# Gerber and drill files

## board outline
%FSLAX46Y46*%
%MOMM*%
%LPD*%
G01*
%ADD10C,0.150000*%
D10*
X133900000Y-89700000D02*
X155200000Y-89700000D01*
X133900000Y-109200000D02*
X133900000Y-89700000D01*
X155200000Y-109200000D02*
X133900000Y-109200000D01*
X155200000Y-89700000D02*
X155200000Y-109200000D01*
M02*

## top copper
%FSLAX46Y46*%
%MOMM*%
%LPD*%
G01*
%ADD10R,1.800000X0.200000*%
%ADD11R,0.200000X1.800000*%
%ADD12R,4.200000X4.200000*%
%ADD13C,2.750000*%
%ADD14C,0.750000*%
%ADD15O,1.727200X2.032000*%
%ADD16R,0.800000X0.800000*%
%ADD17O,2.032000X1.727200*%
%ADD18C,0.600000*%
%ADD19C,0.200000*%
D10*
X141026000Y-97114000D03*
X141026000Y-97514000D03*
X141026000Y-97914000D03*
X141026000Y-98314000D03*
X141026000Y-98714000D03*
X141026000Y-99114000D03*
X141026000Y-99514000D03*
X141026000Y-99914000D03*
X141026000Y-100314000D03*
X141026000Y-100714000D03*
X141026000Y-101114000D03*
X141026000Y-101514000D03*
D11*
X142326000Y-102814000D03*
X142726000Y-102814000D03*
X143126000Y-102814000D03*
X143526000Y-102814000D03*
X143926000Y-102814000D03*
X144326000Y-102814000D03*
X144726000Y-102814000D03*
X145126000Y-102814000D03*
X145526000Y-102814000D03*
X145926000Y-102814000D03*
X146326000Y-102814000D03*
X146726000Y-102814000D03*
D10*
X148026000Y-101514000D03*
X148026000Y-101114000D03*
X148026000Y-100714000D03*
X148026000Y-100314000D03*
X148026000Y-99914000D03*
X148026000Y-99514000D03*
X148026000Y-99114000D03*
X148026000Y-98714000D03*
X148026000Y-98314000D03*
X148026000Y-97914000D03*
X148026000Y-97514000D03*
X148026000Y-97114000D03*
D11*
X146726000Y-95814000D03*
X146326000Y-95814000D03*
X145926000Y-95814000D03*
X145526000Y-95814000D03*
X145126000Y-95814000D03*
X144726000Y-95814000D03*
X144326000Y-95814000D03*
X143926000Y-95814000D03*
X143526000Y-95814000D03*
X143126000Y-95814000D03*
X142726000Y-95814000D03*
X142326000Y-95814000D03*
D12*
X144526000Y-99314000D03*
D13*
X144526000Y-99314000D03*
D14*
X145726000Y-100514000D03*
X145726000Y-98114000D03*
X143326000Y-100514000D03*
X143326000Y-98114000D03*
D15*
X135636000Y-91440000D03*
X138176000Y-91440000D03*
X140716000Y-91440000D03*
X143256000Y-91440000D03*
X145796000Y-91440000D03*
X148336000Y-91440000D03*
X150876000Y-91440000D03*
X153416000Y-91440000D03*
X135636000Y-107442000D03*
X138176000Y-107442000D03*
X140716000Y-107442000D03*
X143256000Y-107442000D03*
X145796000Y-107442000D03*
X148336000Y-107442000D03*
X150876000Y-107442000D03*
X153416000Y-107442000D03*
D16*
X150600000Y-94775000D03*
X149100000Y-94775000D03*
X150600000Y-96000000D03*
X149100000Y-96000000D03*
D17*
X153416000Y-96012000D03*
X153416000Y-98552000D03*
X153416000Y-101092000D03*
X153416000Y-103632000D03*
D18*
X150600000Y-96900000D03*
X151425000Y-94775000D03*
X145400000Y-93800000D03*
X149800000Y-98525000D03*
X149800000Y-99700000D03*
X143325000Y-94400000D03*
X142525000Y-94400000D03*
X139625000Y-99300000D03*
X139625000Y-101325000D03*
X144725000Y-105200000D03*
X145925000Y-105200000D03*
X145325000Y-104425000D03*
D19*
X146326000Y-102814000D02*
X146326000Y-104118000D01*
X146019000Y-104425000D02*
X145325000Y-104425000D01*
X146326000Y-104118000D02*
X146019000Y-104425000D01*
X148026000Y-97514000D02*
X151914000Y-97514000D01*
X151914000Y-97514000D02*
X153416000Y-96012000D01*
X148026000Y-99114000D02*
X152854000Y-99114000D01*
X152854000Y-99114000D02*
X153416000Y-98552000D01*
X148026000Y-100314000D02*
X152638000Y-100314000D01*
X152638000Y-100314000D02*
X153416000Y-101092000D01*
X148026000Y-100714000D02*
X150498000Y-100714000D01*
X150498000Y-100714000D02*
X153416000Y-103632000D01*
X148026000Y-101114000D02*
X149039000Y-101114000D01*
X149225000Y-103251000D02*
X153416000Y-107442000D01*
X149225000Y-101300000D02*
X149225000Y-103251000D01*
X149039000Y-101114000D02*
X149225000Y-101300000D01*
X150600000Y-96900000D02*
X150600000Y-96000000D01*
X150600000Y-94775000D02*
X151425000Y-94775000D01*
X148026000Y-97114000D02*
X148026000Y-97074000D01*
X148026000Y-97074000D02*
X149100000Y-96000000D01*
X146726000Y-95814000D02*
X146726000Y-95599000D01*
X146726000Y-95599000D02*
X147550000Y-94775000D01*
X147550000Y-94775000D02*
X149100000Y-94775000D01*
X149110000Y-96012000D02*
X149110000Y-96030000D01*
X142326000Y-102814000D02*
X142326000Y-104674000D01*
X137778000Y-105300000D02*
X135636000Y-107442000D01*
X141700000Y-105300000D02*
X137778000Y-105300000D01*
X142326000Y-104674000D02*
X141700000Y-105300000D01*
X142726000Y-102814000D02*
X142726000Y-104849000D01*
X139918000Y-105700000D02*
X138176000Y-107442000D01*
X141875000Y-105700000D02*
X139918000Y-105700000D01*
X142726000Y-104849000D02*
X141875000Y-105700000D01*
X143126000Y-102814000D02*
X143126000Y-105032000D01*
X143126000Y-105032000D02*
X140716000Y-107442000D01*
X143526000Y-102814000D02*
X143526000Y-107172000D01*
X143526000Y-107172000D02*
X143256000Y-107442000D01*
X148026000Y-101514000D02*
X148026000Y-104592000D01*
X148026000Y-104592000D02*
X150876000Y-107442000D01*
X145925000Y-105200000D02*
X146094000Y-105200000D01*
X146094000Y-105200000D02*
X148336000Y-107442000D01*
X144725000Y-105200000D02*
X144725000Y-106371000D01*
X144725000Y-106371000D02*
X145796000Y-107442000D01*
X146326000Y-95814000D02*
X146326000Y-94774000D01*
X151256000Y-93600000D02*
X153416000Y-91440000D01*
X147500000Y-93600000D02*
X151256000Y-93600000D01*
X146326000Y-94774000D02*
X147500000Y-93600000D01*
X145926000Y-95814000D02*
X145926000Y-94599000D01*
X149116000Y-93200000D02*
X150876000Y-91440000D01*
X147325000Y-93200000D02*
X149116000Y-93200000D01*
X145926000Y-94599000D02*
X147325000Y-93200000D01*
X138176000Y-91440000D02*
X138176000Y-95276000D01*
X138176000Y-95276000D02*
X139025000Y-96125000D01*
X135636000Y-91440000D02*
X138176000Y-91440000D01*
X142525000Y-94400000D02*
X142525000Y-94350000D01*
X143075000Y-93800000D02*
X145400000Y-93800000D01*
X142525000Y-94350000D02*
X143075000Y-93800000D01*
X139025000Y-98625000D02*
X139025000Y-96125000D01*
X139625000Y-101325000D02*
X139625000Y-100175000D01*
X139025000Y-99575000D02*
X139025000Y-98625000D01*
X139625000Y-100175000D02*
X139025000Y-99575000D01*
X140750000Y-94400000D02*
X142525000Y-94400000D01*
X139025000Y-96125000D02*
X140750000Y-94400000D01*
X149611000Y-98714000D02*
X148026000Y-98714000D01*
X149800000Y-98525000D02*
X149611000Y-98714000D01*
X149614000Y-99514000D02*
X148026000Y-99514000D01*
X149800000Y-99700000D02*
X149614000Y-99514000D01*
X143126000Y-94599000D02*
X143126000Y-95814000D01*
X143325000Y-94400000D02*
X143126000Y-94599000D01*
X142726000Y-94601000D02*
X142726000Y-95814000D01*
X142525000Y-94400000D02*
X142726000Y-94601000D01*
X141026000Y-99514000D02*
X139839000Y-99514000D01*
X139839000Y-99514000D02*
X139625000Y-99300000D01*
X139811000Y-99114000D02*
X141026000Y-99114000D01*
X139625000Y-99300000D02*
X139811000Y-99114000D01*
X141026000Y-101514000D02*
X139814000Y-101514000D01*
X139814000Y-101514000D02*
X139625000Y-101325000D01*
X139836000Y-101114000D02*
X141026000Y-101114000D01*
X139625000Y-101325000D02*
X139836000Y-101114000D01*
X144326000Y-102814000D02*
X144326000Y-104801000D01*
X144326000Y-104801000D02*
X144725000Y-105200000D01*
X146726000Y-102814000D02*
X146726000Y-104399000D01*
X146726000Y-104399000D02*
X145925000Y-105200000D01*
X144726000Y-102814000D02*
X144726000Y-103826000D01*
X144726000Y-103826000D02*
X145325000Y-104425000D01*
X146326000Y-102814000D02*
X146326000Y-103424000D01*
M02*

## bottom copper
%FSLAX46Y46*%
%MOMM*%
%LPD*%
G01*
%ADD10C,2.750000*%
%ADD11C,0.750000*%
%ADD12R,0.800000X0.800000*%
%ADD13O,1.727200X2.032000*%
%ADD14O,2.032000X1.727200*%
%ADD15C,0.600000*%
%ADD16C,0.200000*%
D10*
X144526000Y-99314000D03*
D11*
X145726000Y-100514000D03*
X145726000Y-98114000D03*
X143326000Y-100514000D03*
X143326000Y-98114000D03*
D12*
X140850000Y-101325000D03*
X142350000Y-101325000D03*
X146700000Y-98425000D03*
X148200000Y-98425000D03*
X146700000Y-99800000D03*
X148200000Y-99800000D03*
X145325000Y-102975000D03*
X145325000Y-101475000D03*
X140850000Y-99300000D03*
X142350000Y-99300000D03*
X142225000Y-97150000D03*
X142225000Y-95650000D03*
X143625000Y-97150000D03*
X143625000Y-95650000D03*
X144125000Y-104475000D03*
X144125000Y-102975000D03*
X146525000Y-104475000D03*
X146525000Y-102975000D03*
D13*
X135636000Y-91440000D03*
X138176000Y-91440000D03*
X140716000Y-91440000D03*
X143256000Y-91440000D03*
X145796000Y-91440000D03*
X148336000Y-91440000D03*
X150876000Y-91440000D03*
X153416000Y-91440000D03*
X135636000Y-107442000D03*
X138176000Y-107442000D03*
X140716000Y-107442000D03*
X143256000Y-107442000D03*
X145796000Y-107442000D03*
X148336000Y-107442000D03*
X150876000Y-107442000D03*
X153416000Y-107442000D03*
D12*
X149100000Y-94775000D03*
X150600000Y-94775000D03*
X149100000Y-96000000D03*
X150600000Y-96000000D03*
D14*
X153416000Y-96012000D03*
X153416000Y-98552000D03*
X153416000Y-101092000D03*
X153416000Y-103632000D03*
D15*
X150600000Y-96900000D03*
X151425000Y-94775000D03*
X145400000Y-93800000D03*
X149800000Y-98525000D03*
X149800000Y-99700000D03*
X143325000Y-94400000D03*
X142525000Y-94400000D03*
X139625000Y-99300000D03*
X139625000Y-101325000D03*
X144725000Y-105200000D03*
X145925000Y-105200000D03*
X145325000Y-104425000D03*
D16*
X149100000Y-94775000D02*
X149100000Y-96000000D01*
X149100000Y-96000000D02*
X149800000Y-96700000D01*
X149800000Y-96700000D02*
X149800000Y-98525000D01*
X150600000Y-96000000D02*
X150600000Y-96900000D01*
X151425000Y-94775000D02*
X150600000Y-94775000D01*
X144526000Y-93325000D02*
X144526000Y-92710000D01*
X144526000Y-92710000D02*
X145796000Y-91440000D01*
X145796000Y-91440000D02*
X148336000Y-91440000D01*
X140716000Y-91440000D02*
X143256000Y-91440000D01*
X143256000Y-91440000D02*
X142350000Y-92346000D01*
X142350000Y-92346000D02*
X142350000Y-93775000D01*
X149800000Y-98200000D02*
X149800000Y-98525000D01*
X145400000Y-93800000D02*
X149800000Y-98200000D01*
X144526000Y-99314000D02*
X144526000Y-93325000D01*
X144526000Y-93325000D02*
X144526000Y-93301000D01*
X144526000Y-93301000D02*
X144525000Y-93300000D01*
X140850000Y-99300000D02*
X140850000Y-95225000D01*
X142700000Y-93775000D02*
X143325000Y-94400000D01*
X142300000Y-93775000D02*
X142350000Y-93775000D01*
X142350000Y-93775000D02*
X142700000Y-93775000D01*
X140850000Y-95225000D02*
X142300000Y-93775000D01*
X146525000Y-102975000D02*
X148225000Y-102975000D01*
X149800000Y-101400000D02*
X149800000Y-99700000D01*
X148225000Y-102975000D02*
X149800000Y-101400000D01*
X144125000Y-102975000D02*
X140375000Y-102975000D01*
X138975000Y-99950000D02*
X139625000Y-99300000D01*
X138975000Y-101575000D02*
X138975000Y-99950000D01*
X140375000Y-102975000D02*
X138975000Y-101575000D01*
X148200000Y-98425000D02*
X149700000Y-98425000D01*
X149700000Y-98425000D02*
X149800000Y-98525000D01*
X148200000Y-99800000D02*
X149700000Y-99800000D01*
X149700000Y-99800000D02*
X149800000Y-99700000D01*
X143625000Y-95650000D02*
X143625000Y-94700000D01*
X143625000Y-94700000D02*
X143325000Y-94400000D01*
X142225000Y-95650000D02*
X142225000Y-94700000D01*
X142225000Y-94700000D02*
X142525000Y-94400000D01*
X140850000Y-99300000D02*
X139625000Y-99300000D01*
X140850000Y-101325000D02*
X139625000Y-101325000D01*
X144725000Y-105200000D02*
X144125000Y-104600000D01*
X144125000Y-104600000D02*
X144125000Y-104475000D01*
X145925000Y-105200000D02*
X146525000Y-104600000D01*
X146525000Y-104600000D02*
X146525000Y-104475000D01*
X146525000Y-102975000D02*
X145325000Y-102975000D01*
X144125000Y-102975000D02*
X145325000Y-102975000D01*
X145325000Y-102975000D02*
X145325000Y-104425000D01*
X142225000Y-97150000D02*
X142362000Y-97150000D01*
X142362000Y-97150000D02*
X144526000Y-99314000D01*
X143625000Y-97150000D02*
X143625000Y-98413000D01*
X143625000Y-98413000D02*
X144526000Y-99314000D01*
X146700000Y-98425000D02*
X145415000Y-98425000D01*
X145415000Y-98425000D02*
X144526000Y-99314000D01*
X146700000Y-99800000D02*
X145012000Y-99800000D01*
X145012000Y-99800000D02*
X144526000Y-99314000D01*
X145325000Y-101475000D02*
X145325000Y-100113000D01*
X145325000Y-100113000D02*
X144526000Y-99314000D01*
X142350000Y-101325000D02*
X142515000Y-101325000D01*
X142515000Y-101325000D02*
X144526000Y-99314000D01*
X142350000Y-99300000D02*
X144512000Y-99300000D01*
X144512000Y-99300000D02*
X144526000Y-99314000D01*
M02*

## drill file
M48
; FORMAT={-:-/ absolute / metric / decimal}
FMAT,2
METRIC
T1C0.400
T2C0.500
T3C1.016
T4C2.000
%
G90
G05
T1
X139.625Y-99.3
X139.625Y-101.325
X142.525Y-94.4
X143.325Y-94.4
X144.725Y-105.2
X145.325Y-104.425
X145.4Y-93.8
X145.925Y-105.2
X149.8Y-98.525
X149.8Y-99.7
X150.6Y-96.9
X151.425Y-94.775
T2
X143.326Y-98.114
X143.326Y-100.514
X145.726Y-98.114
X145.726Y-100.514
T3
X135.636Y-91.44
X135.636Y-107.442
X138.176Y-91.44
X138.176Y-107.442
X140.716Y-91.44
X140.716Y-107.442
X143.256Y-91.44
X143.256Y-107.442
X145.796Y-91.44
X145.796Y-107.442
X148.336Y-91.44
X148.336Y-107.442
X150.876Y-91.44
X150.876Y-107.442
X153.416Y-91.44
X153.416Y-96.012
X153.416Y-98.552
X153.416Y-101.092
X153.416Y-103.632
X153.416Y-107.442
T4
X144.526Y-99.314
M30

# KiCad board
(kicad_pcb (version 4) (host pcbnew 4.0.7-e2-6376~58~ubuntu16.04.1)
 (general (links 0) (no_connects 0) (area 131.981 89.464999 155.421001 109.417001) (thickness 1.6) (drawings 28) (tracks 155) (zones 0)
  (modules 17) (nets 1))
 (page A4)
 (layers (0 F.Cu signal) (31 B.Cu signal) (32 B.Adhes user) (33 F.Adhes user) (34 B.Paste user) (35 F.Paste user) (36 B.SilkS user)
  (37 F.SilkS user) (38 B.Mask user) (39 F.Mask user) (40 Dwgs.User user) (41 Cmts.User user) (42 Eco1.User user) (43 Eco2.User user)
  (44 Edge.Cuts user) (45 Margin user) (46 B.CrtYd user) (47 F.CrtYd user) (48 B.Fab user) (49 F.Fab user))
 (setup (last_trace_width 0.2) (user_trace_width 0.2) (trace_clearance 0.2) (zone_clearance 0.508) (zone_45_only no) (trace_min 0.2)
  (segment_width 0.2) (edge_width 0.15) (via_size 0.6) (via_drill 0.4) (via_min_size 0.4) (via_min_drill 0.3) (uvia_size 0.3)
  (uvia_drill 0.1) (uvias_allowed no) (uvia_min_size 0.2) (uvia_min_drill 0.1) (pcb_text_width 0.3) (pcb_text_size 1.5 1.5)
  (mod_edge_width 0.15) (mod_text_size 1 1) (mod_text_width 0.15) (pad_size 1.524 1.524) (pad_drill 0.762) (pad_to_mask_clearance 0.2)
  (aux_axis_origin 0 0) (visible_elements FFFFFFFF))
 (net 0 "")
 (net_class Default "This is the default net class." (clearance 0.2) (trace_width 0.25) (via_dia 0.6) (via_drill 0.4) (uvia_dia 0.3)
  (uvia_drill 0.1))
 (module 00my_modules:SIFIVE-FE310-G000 (layer F.Cu) (at 144.526 99.314)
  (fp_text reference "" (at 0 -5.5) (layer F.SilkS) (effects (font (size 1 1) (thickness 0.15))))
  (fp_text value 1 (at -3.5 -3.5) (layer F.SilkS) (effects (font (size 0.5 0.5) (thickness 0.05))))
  (pad DQ3 smd rect (at -3.5 -2.2) (size 1.8 0.2) (layers F.Cu F.Paste F.Mask))
  (pad DQ2 smd rect (at -3.5 -1.8) (size 1.8 0.2) (layers F.Cu F.Paste F.Mask))
  (pad DQ1 smd rect (at -3.5 -1.4) (size 1.8 0.2) (layers F.Cu F.Paste F.Mask))
  (pad DQ0 smd rect (at -3.5 -1) (size 1.8 0.2) (layers F.Cu F.Paste F.Mask))
  (pad CS smd rect (at -3.5 -0.6) (size 1.8 0.2) (layers F.Cu F.Paste F.Mask))
  (pad 1.8V smd rect (at -3.5 -0.2) (size 1.8 0.2) (layers F.Cu F.Paste F.Mask))
  (pad 1.8V smd rect (at -3.5 0.2) (size 1.8 0.2) (layers F.Cu F.Paste F.Mask))
  (pad PLL smd rect (at -3.5 0.6) (size 1.8 0.2) (layers F.Cu F.Paste F.Mask))
  (pad XIN smd rect (at -3.5 1) (size 1.8 0.2) (layers F.Cu F.Paste F.Mask))
  (pad NC smd rect (at -3.5 1.4) (size 1.8 0.2) (layers F.Cu F.Paste F.Mask))
  (pad 3.3V smd rect (at -3.5 1.8) (size 1.8 0.2) (layers F.Cu F.Paste F.Mask))
  (pad 3.3V smd rect (at -3.5 2.2) (size 1.8 0.2) (layers F.Cu F.Paste F.Mask))
  (pad TCK smd rect (at -2.2 3.5 90) (size 1.8 0.2) (layers F.Cu F.Paste F.Mask))
  (pad TDO smd rect (at -1.8 3.5 90) (size 1.8 0.2) (layers F.Cu F.Paste F.Mask))
  (pad TMS smd rect (at -1.4 3.5 90) (size 1.8 0.2) (layers F.Cu F.Paste F.Mask))
  (pad TDI smd rect (at -1 3.5 90) (size 1.8 0.2) (layers F.Cu F.Paste F.Mask))
  (pad 17 smd rect (at -0.6 3.5 90) (size 1.8 0.2) (layers F.Cu F.Paste F.Mask))
  (pad WAKE smd rect (at -0.2 3.5 90) (size 1.8 0.2) (layers F.Cu F.Paste F.Mask))
  (pad 1.8V smd rect (at 0.2 3.5 90) (size 1.8 0.2) (layers F.Cu F.Paste F.Mask))
  (pad 20 smd rect (at 0.6 3.5 90) (size 1.8 0.2) (layers F.Cu F.Paste F.Mask))
  (pad 21 smd rect (at 1 3.5 90) (size 1.8 0.2) (layers F.Cu F.Paste F.Mask))
  (pad 22 smd rect (at 1.4 3.5 90) (size 1.8 0.2) (layers F.Cu F.Paste F.Mask))
  (pad 1.8V smd rect (at 1.8 3.5 90) (size 1.8 0.2) (layers F.Cu F.Paste F.Mask))
  (pad ERST smd rect (at 2.2 3.5 90) (size 1.8 0.2) (layers F.Cu F.Paste F.Mask))
  (pad G00 smd rect (at 3.5 2.2) (size 1.8 0.2) (layers F.Cu F.Paste F.Mask))
  (pad G01 smd rect (at 3.5 1.8) (size 1.8 0.2) (layers F.Cu F.Paste F.Mask))
  (pad G02 smd rect (at 3.5 1.4) (size 1.8 0.2) (layers F.Cu F.Paste F.Mask))
  (pad G03 smd rect (at 3.5 1) (size 1.8 0.2) (layers F.Cu F.Paste F.Mask))
  (pad G04 smd rect (at 3.5 0.6) (size 1.8 0.2) (layers F.Cu F.Paste F.Mask))
  (pad 1.8V smd rect (at 3.5 0.2) (size 1.8 0.2) (layers F.Cu F.Paste F.Mask))
  (pad G05 smd rect (at 3.5 -0.2) (size 1.8 0.2) (layers F.Cu F.Paste F.Mask))
  (pad 3.3V smd rect (at 3.5 -0.6) (size 1.8 0.2) (layers F.Cu F.Paste F.Mask))
  (pad G09 smd rect (at 3.5 -1) (size 1.8 0.2) (layers F.Cu F.Paste F.Mask))
  (pad G10 smd rect (at 3.5 -1.4) (size 1.8 0.2) (layers F.Cu F.Paste F.Mask))
  (pad G11 smd rect (at 3.5 -1.8) (size 1.8 0.2) (layers F.Cu F.Paste F.Mask))
  (pad G12 smd rect (at 3.5 -2.2) (size 1.8 0.2) (layers F.Cu F.Paste F.Mask))
  (pad G13 smd rect (at 2.2 -3.5 90) (size 1.8 0.2) (layers F.Cu F.Paste F.Mask))
  (pad RX smd rect (at 1.8 -3.5 90) (size 1.8 0.2) (layers F.Cu F.Paste F.Mask))
  (pad TX smd rect (at 1.4 -3.5 90) (size 1.8 0.2) (layers F.Cu F.Paste F.Mask))
  (pad G18 smd rect (at 1 -3.5 90) (size 1.8 0.2) (layers F.Cu F.Paste F.Mask))
  (pad G19 smd rect (at 0.6 -3.5 90) (size 1.8 0.2) (layers F.Cu F.Paste F.Mask))
  (pad G20 smd rect (at 0.2 -3.5 90) (size 1.8 0.2) (layers F.Cu F.Paste F.Mask))
  (pad G21 smd rect (at -0.2 -3.5 90) (size 1.8 0.2) (layers F.Cu F.Paste F.Mask))
  (pad G22 smd rect (at -0.6 -3.5 90) (size 1.8 0.2) (layers F.Cu F.Paste F.Mask))
  (pad G23 smd rect (at -1 -3.5 90) (size 1.8 0.2) (layers F.Cu F.Paste F.Mask))
  (pad 1.8V smd rect (at -1.4 -3.5 90) (size 1.8 0.2) (layers F.Cu F.Paste F.Mask))
  (pad 3.3V smd rect (at -1.8 -3.5 90) (size 1.8 0.2) (layers F.Cu F.Paste F.Mask))
  (pad SCK smd rect (at -2.2 -3.5 90) (size 1.8 0.2) (layers F.Cu F.Paste F.Mask))
  (pad GND smd rect (at 0 0) (size 4.2 4.2) (layers F.Cu F.Paste F.Mask))
  (pad "" thru_hole circle (at 0 0) (size 2.75 2.75) (drill 2) (layers *.Cu *.Mask F.SilkS))
  (pad "" thru_hole circle (at 1.2 1.2) (size 0.75 0.75) (drill 0.5) (layers *.Cu *.Mask F.SilkS))
  (pad "" thru_hole circle (at 1.2 -1.2) (size 0.75 0.75) (drill 0.5) (layers *.Cu *.Mask F.SilkS))
  (pad "" thru_hole circle (at -1.2 1.2) (size 0.75 0.75) (drill 0.5) (layers *.Cu *.Mask F.SilkS))
  (pad "" thru_hole circle (at -1.2 -1.2) (size 0.75 0.75) (drill 0.5) (layers *.Cu *.Mask F.SilkS)))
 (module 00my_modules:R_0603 (layer B.Cu) (at 141.6 101.325)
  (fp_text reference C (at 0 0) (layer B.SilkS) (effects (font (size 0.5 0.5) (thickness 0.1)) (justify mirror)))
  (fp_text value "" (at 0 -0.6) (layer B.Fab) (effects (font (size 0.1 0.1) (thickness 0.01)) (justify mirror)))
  (pad 1 smd rect (at -0.75 0) (size 0.8 0.8) (layers B.Cu B.Paste B.Mask))
  (pad 2 smd rect (at 0.75 0) (size 0.8 0.8) (layers B.Cu B.Paste B.Mask)))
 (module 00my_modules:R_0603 (layer B.Cu) (at 147.45 98.425)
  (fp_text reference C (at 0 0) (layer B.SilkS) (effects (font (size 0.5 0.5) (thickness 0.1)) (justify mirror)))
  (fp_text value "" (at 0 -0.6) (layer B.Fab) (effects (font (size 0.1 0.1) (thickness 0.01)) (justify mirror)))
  (pad 1 smd rect (at -0.75 0) (size 0.8 0.8) (layers B.Cu B.Paste B.Mask))
  (pad 2 smd rect (at 0.75 0) (size 0.8 0.8) (layers B.Cu B.Paste B.Mask)))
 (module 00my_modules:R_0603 (layer B.Cu) (at 147.45 99.8)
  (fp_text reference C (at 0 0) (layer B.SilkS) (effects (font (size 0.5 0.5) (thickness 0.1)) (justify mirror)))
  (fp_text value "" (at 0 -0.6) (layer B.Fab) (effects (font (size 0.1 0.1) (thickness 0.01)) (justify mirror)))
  (pad 1 smd rect (at -0.75 0) (size 0.8 0.8) (layers B.Cu B.Paste B.Mask))
  (pad 2 smd rect (at 0.75 0) (size 0.8 0.8) (layers B.Cu B.Paste B.Mask)))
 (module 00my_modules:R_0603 (layer B.Cu) (at 145.325 102.225 90)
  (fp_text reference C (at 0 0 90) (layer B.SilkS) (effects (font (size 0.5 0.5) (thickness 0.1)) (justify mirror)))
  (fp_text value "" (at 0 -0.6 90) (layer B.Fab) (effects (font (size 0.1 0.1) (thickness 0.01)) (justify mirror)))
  (pad 1 smd rect (at -0.75 0 90) (size 0.8 0.8) (layers B.Cu B.Paste B.Mask))
  (pad 2 smd rect (at 0.75 0 90) (size 0.8 0.8) (layers B.Cu B.Paste B.Mask)))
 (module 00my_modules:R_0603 (layer B.Cu) (at 141.6 99.3)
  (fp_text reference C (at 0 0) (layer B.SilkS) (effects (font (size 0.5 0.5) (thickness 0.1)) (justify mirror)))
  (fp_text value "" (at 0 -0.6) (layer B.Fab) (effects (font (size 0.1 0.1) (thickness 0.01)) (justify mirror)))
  (pad 1 smd rect (at -0.75 0) (size 0.8 0.8) (layers B.Cu B.Paste B.Mask))
  (pad 2 smd rect (at 0.75 0) (size 0.8 0.8) (layers B.Cu B.Paste B.Mask)))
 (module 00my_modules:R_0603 (layer B.Cu) (at 142.225 96.4 90)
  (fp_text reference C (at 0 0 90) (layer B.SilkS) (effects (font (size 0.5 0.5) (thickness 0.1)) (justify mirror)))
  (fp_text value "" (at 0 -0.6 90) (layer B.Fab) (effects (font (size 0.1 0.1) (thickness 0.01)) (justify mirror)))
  (pad 1 smd rect (at -0.75 0 90) (size 0.8 0.8) (layers B.Cu B.Paste B.Mask))
  (pad 2 smd rect (at 0.75 0 90) (size 0.8 0.8) (layers B.Cu B.Paste B.Mask)))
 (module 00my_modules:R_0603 (layer B.Cu) (at 143.625 96.4 90)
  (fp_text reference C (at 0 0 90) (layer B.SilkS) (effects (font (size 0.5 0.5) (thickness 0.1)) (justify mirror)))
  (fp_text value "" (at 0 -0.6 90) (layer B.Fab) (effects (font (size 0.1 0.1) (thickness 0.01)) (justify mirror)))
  (pad 1 smd rect (at -0.75 0 90) (size 0.8 0.8) (layers B.Cu B.Paste B.Mask))
  (pad 2 smd rect (at 0.75 0 90) (size 0.8 0.8) (layers B.Cu B.Paste B.Mask)))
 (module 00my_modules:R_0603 (layer B.Cu) (at 144.125 103.725 90)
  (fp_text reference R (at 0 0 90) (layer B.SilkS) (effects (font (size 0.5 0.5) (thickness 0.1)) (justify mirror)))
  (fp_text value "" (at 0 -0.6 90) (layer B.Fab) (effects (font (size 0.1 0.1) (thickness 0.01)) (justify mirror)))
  (pad 1 smd rect (at -0.75 0 90) (size 0.8 0.8) (layers B.Cu B.Paste B.Mask))
  (pad 2 smd rect (at 0.75 0 90) (size 0.8 0.8) (layers B.Cu B.Paste B.Mask)))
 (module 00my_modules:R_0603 (layer B.Cu) (at 146.525 103.725 90)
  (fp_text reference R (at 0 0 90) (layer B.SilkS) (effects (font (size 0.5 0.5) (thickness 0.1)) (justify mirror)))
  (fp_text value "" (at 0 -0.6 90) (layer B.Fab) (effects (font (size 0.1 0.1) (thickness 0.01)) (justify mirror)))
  (pad 1 smd rect (at -0.75 0 90) (size 0.8 0.8) (layers B.Cu B.Paste B.Mask))
  (pad 2 smd rect (at 0.75 0 90) (size 0.8 0.8) (layers B.Cu B.Paste B.Mask)))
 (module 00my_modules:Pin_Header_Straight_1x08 (layer F.Cu) (at 135.636 91.44 90)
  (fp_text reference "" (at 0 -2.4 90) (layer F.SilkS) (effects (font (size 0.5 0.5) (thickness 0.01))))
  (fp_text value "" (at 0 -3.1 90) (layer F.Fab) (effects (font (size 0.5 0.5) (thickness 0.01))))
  (pad 1 thru_hole oval (at 0 0 90) (size 2.032 1.7272) (drill 1.016) (layers *.Cu *.Mask F.SilkS))
  (pad 2 thru_hole oval (at 0 2.54 90) (size 2.032 1.7272) (drill 1.016) (layers *.Cu *.Mask F.SilkS))
  (pad 3 thru_hole oval (at 0 5.08 90) (size 2.032 1.7272) (drill 1.016) (layers *.Cu *.Mask F.SilkS))
  (pad 4 thru_hole oval (at 0 7.62 90) (size 2.032 1.7272) (drill 1.016) (layers *.Cu *.Mask F.SilkS))
  (pad 5 thru_hole oval (at 0 10.16 90) (size 2.032 1.7272) (drill 1.016) (layers *.Cu *.Mask F.SilkS))
  (pad 6 thru_hole oval (at 0 12.7 90) (size 2.032 1.7272) (drill 1.016) (layers *.Cu *.Mask F.SilkS))
  (pad 7 thru_hole oval (at 0 15.24 90) (size 2.032 1.7272) (drill 1.016) (layers *.Cu *.Mask F.SilkS))
  (pad 8 thru_hole oval (at 0 17.78 90) (size 2.032 1.7272) (drill 1.016) (layers *.Cu *.Mask F.SilkS)))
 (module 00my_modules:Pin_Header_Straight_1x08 (layer F.Cu) (at 135.636 107.442 90)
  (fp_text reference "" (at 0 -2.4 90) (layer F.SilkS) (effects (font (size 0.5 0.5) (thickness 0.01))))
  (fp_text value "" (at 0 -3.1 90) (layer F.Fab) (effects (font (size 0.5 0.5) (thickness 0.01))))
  (pad 1 thru_hole oval (at 0 0 90) (size 2.032 1.7272) (drill 1.016) (layers *.Cu *.Mask F.SilkS))
  (pad 2 thru_hole oval (at 0 2.54 90) (size 2.032 1.7272) (drill 1.016) (layers *.Cu *.Mask F.SilkS))
  (pad 3 thru_hole oval (at 0 5.08 90) (size 2.032 1.7272) (drill 1.016) (layers *.Cu *.Mask F.SilkS))
  (pad 4 thru_hole oval (at 0 7.62 90) (size 2.032 1.7272) (drill 1.016) (layers *.Cu *.Mask F.SilkS))
  (pad 5 thru_hole oval (at 0 10.16 90) (size 2.032 1.7272) (drill 1.016) (layers *.Cu *.Mask F.SilkS))
  (pad 6 thru_hole oval (at 0 12.7 90) (size 2.032 1.7272) (drill 1.016) (layers *.Cu *.Mask F.SilkS))
  (pad 7 thru_hole oval (at 0 15.24 90) (size 2.032 1.7272) (drill 1.016) (layers *.Cu *.Mask F.SilkS))
  (pad 8 thru_hole oval (at 0 17.78 90) (size 2.032 1.7272) (drill 1.016) (layers *.Cu *.Mask F.SilkS)))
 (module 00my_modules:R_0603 (layer B.Cu) (at 149.85 94.775)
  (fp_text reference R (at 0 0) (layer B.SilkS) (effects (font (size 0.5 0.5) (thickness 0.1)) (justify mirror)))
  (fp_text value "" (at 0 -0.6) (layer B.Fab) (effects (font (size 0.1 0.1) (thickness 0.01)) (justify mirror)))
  (pad 1 smd rect (at -0.75 0) (size 0.8 0.8) (layers B.Cu B.Paste B.Mask))
  (pad 2 smd rect (at 0.75 0) (size 0.8 0.8) (layers B.Cu B.Paste B.Mask)))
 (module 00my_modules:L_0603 (layer F.Cu) (at 149.85 94.775 180)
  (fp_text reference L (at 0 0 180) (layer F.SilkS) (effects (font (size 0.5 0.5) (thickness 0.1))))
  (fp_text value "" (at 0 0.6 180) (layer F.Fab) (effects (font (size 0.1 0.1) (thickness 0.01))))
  (pad 1 smd rect (at -0.75 0 180) (size 0.8 0.8) (layers F.Cu F.Paste F.Mask))
  (pad 2 smd rect (at 0.75 0 180) (size 0.8 0.8) (layers F.Cu F.Paste F.Mask)))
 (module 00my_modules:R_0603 (layer B.Cu) (at 149.85 96)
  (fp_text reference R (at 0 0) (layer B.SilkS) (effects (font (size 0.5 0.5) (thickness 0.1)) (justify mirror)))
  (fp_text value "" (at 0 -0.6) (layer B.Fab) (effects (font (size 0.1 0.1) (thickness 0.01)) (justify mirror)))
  (pad 1 smd rect (at -0.75 0) (size 0.8 0.8) (layers B.Cu B.Paste B.Mask))
  (pad 2 smd rect (at 0.75 0) (size 0.8 0.8) (layers B.Cu B.Paste B.Mask)))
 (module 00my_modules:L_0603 (layer F.Cu) (at 149.85 96 180)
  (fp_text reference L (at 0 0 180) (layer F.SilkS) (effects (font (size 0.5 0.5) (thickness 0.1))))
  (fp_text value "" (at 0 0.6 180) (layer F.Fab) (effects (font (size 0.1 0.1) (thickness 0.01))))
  (pad 1 smd rect (at -0.75 0 180) (size 0.8 0.8) (layers F.Cu F.Paste F.Mask))
  (pad 2 smd rect (at 0.75 0 180) (size 0.8 0.8) (layers F.Cu F.Paste F.Mask)))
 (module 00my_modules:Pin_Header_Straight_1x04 (layer F.Cu) (at 153.416 96.012)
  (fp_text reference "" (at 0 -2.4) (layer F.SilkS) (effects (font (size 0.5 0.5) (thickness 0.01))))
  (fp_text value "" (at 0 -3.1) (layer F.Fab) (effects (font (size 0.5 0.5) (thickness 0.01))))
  (pad 1 thru_hole oval (at 0 0) (size 2.032 1.7272) (drill 1.016) (layers *.Cu *.Mask F.SilkS))
  (pad 2 thru_hole oval (at 0 2.54) (size 2.032 1.7272) (drill 1.016) (layers *.Cu *.Mask F.SilkS))
  (pad 3 thru_hole oval (at 0 5.08) (size 2.032 1.7272) (drill 1.016) (layers *.Cu *.Mask F.SilkS))
  (pad 4 thru_hole oval (at 0 7.62) (size 2.032 1.7272) (drill 1.016) (layers *.Cu *.Mask F.SilkS)))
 (gr_line (start 133.9 89.7) (end 155.2 89.7) (angle 90) (layer Edge.Cuts) (width 0.15))
 (gr_line (start 133.9 109.2) (end 133.9 89.7) (angle 90) (layer Edge.Cuts) (width 0.15))
 (gr_line (start 155.2 109.2) (end 133.9 109.2) (angle 90) (layer Edge.Cuts) (width 0.15))
 (gr_line (start 155.2 89.7) (end 155.2 109.2) (angle 90) (layer Edge.Cuts) (width 0.15))
 (segment (start 146.326 102.814) (end 146.326 104.118) (width 0.2) (layer F.Cu) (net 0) (status 400000))
 (segment (start 146.019 104.425) (end 145.325 104.425) (width 0.2) (layer F.Cu) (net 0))
 (segment (start 146.326 104.118) (end 146.019 104.425) (width 0.2) (layer F.Cu) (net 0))
 (segment (start 148.026 97.514) (end 151.914 97.514) (width 0.2) (layer F.Cu) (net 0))
 (segment (start 151.914 97.514) (end 153.416 96.012) (width 0.2) (layer F.Cu) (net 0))
 (segment (start 148.026 99.114) (end 152.854 99.114) (width 0.2) (layer F.Cu) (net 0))
 (segment (start 152.854 99.114) (end 153.416 98.552) (width 0.2) (layer F.Cu) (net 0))
 (segment (start 148.026 100.314) (end 152.638 100.314) (width 0.2) (layer F.Cu) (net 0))
 (segment (start 152.638 100.314) (end 153.416 101.092) (width 0.2) (layer F.Cu) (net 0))
 (segment (start 148.026 100.714) (end 150.498 100.714) (width 0.2) (layer F.Cu) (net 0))
 (segment (start 150.498 100.714) (end 153.416 103.632) (width 0.2) (layer F.Cu) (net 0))
 (segment (start 148.026 101.114) (end 149.039 101.114) (width 0.2) (layer F.Cu) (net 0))
 (segment (start 149.225 103.251) (end 153.416 107.442) (width 0.2) (layer F.Cu) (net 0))
 (segment (start 149.225 101.3) (end 149.225 103.251) (width 0.2) (layer F.Cu) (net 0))
 (segment (start 149.039 101.114) (end 149.225 101.3) (width 0.2) (layer F.Cu) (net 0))
 (segment (start 149.1 94.775) (end 149.1 96) (width 0.2) (layer B.Cu) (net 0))
 (segment (start 149.1 96) (end 149.8 96.7) (width 0.2) (layer B.Cu) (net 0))
 (segment (start 149.8 96.7) (end 149.8 98.525) (width 0.2) (layer B.Cu) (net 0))
 (segment (start 150.6 96) (end 150.6 96.9) (width 0.2) (layer B.Cu) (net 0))
 (segment (start 150.6 96.9) (end 150.6 96) (width 0.2) (layer F.Cu) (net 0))
 (via (at 150.6 96.9) (size 0.6) (drill 0.4) (layers F.Cu B.Cu) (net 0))
 (segment (start 150.6 94.775) (end 151.425 94.775) (width 0.2) (layer F.Cu) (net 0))
 (segment (start 151.425 94.775) (end 150.6 94.775) (width 0.2) (layer B.Cu) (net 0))
 (via (at 151.425 94.775) (size 0.6) (drill 0.4) (layers F.Cu B.Cu) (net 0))
 (segment (start 148.026 97.114) (end 148.026 97.074) (width 0.2) (layer F.Cu) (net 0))
 (segment (start 148.026 97.074) (end 149.1 96) (width 0.2) (layer F.Cu) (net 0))
 (segment (start 146.726 95.814) (end 146.726 95.599) (width 0.2) (layer F.Cu) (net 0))
 (segment (start 146.726 95.599) (end 147.55 94.775) (width 0.2) (layer F.Cu) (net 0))
 (segment (start 147.55 94.775) (end 149.1 94.775) (width 0.2) (layer F.Cu) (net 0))
 (segment (start 149.11 96.012) (end 149.11 96.03) (width 0.2) (layer F.Cu) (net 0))
 (segment (start 142.326 102.814) (end 142.326 104.674) (width 0.2) (layer F.Cu) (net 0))
 (segment (start 137.778 105.3) (end 135.636 107.442) (width 0.2) (layer F.Cu) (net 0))
 (segment (start 141.7 105.3) (end 137.778 105.3) (width 0.2) (layer F.Cu) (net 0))
 (segment (start 142.326 104.674) (end 141.7 105.3) (width 0.2) (layer F.Cu) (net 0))
 (segment (start 142.726 102.814) (end 142.726 104.849) (width 0.2) (layer F.Cu) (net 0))
 (segment (start 139.918 105.7) (end 138.176 107.442) (width 0.2) (layer F.Cu) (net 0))
 (segment (start 141.875 105.7) (end 139.918 105.7) (width 0.2) (layer F.Cu) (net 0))
 (segment (start 142.726 104.849) (end 141.875 105.7) (width 0.2) (layer F.Cu) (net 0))
 (segment (start 143.126 102.814) (end 143.126 105.032) (width 0.2) (layer F.Cu) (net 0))
 (segment (start 143.126 105.032) (end 140.716 107.442) (width 0.2) (layer F.Cu) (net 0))
 (segment (start 143.526 102.814) (end 143.526 107.172) (width 0.2) (layer F.Cu) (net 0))
 (segment (start 143.526 107.172) (end 143.256 107.442) (width 0.2) (layer F.Cu) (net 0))
 (segment (start 148.026 101.514) (end 148.026 104.592) (width 0.2) (layer F.Cu) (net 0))
 (segment (start 148.026 104.592) (end 150.876 107.442) (width 0.2) (layer F.Cu) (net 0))
 (segment (start 145.925 105.2) (end 146.094 105.2) (width 0.2) (layer F.Cu) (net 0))
 (segment (start 146.094 105.2) (end 148.336 107.442) (width 0.2) (layer F.Cu) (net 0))
 (segment (start 144.725 105.2) (end 144.725 106.371) (width 0.2) (layer F.Cu) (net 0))
 (segment (start 144.725 106.371) (end 145.796 107.442) (width 0.2) (layer F.Cu) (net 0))
 (segment (start 146.326 95.814) (end 146.326 94.774) (width 0.2) (layer F.Cu) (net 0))
 (segment (start 151.256 93.6) (end 153.416 91.44) (width 0.2) (layer F.Cu) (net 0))
 (segment (start 147.5 93.6) (end 151.256 93.6) (width 0.2) (layer F.Cu) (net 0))
 (segment (start 146.326 94.774) (end 147.5 93.6) (width 0.2) (layer F.Cu) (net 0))
 (segment (start 145.926 95.814) (end 145.926 94.599) (width 0.2) (layer F.Cu) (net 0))
 (segment (start 149.116 93.2) (end 150.876 91.44) (width 0.2) (layer F.Cu) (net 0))
 (segment (start 147.325 93.2) (end 149.116 93.2) (width 0.2) (layer F.Cu) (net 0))
 (segment (start 145.926 94.599) (end 147.325 93.2) (width 0.2) (layer F.Cu) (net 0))
 (segment (start 144.526 93.325) (end 144.526 92.71) (width 0.2) (layer B.Cu) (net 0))
 (segment (start 144.526 92.71) (end 145.796 91.44) (width 0.2) (layer B.Cu) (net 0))
 (segment (start 145.796 91.44) (end 148.336 91.44) (width 0.2) (layer B.Cu) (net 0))
 (segment (start 140.716 91.44) (end 143.256 91.44) (width 0.2) (layer B.Cu) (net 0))
 (segment (start 143.256 91.44) (end 142.35 92.346) (width 0.2) (layer B.Cu) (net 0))
 (segment (start 142.35 92.346) (end 142.35 93.775) (width 0.2) (layer B.Cu) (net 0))
 (segment (start 138.176 91.44) (end 138.176 95.276) (width 0.2) (layer F.Cu) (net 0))
 (segment (start 138.176 95.276) (end 139.025 96.125) (width 0.2) (layer F.Cu) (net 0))
 (segment (start 135.636 91.44) (end 138.176 91.44) (width 0.2) (layer F.Cu) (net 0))
 (segment (start 142.525 94.4) (end 142.525 94.35) (width 0.2) (layer F.Cu) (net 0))
 (segment (start 149.8 98.2) (end 149.8 98.525) (width 0.2) (layer B.Cu) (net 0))
 (segment (start 145.4 93.8) (end 149.8 98.2) (width 0.2) (layer B.Cu) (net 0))
 (via (at 145.4 93.8) (size 0.6) (drill 0.4) (layers F.Cu B.Cu) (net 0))
 (segment (start 143.075 93.8) (end 145.4 93.8) (width 0.2) (layer F.Cu) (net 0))
 (segment (start 142.525 94.35) (end 143.075 93.8) (width 0.2) (layer F.Cu) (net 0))
 (segment (start 144.526 99.314) (end 144.526 93.325) (width 0.2) (layer B.Cu) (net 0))
 (segment (start 144.526 93.325) (end 144.526 93.301) (width 0.2) (layer B.Cu) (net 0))
 (segment (start 144.526 93.301) (end 144.525 93.3) (width 0.2) (layer B.Cu) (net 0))
 (segment (start 139.025 98.625) (end 139.025 96.125) (width 0.2) (layer F.Cu) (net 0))
 (segment (start 139.625 101.325) (end 139.625 100.175) (width 0.2) (layer F.Cu) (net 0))
 (segment (start 139.025 99.575) (end 139.025 98.625) (width 0.2) (layer F.Cu) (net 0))
 (segment (start 139.625 100.175) (end 139.025 99.575) (width 0.2) (layer F.Cu) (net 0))
 (segment (start 140.75 94.4) (end 142.525 94.4) (width 0.2) (layer F.Cu) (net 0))
 (segment (start 139.025 96.125) (end 140.75 94.4) (width 0.2) (layer F.Cu) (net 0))
 (segment (start 140.85 99.3) (end 140.85 95.225) (width 0.2) (layer B.Cu) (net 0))
 (segment (start 142.7 93.775) (end 143.325 94.4) (width 0.2) (layer B.Cu) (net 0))
 (segment (start 142.3 93.775) (end 142.35 93.775) (width 0.2) (layer B.Cu) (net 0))
 (segment (start 142.35 93.775) (end 142.7 93.775) (width 0.2) (layer B.Cu) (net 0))
 (segment (start 140.85 95.225) (end 142.3 93.775) (width 0.2) (layer B.Cu) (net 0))
 (segment (start 146.525 102.975) (end 148.225 102.975) (width 0.2) (layer B.Cu) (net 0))
 (segment (start 149.8 101.4) (end 149.8 99.7) (width 0.2) (layer B.Cu) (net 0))
 (segment (start 148.225 102.975) (end 149.8 101.4) (width 0.2) (layer B.Cu) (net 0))
 (segment (start 144.125 102.975) (end 140.375 102.975) (width 0.2) (layer B.Cu) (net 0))
 (segment (start 138.975 99.95) (end 139.625 99.3) (width 0.2) (layer B.Cu) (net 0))
 (segment (start 138.975 101.575) (end 138.975 99.95) (width 0.2) (layer B.Cu) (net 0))
 (segment (start 140.375 102.975) (end 138.975 101.575) (width 0.2) (layer B.Cu) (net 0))
 (segment (start 148.2 98.425) (end 149.7 98.425) (width 0.2) (layer B.Cu) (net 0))
 (segment (start 149.7 98.425) (end 149.8 98.525) (width 0.2) (layer B.Cu) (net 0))
 (segment (start 149.611 98.714) (end 148.026 98.714) (width 0.2) (layer F.Cu) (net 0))
 (segment (start 149.8 98.525) (end 149.611 98.714) (width 0.2) (layer F.Cu) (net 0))
 (via (at 149.8 98.525) (size 0.6) (drill 0.4) (layers F.Cu B.Cu) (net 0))
 (segment (start 148.2 99.8) (end 149.7 99.8) (width 0.2) (layer B.Cu) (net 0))
 (segment (start 149.7 99.8) (end 149.8 99.7) (width 0.2) (layer B.Cu) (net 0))
 (segment (start 149.614 99.514) (end 148.026 99.514) (width 0.2) (layer F.Cu) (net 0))
 (via (at 149.8 99.7) (size 0.6) (drill 0.4) (layers F.Cu B.Cu) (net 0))
 (segment (start 149.8 99.7) (end 149.614 99.514) (width 0.2) (layer F.Cu) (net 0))
 (segment (start 143.625 95.65) (end 143.625 94.7) (width 0.2) (layer B.Cu) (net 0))
 (segment (start 143.625 94.7) (end 143.325 94.4) (width 0.2) (layer B.Cu) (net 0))
 (segment (start 143.126 94.599) (end 143.126 95.814) (width 0.2) (layer F.Cu) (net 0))
 (via (at 143.325 94.4) (size 0.6) (drill 0.4) (layers F.Cu B.Cu) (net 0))
 (segment (start 143.325 94.4) (end 143.126 94.599) (width 0.2) (layer F.Cu) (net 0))
 (segment (start 142.225 95.65) (end 142.225 94.7) (width 0.2) (layer B.Cu) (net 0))
 (segment (start 142.225 94.7) (end 142.525 94.4) (width 0.2) (layer B.Cu) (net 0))
 (via (at 142.525 94.4) (size 0.6) (drill 0.4) (layers F.Cu B.Cu) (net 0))
 (segment (start 142.726 94.601) (end 142.726 95.814) (width 0.2) (layer F.Cu) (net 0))
 (segment (start 142.525 94.4) (end 142.726 94.601) (width 0.2) (layer F.Cu) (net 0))
 (segment (start 141.026 99.514) (end 139.839 99.514) (width 0.2) (layer F.Cu) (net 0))
 (segment (start 139.839 99.514) (end 139.625 99.3) (width 0.2) (layer F.Cu) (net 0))
 (segment (start 140.85 99.3) (end 139.625 99.3) (width 0.2) (layer B.Cu) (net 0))
 (segment (start 139.811 99.114) (end 141.026 99.114) (width 0.2) (layer F.Cu) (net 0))
 (segment (start 139.625 99.3) (end 139.811 99.114) (width 0.2) (layer F.Cu) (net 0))
 (via (at 139.625 99.3) (size 0.6) (drill 0.4) (layers F.Cu B.Cu) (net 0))
 (segment (start 141.026 101.514) (end 139.814 101.514) (width 0.2) (layer F.Cu) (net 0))
 (segment (start 139.814 101.514) (end 139.625 101.325) (width 0.2) (layer F.Cu) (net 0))
 (segment (start 140.85 101.325) (end 139.625 101.325) (width 0.2) (layer B.Cu) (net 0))
 (segment (start 139.836 101.114) (end 141.026 101.114) (width 0.2) (layer F.Cu) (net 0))
 (segment (start 139.625 101.325) (end 139.836 101.114) (width 0.2) (layer F.Cu) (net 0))
 (via (at 139.625 101.325) (size 0.6) (drill 0.4) (layers F.Cu B.Cu) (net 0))
 (segment (start 144.326 102.814) (end 144.326 104.801) (width 0.2) (layer F.Cu) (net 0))
 (segment (start 144.725 105.2) (end 144.125 104.6) (width 0.2) (layer B.Cu) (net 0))
 (via (at 144.725 105.2) (size 0.6) (drill 0.4) (layers F.Cu B.Cu) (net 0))
 (segment (start 144.326 104.801) (end 144.725 105.2) (width 0.2) (layer F.Cu) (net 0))
 (segment (start 144.125 104.6) (end 144.125 104.475) (width 0.2) (layer B.Cu) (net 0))
 (segment (start 146.726 102.814) (end 146.726 104.399) (width 0.2) (layer F.Cu) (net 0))
 (segment (start 145.925 105.2) (end 146.525 104.6) (width 0.2) (layer B.Cu) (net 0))
 (via (at 145.925 105.2) (size 0.6) (drill 0.4) (layers F.Cu B.Cu) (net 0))
 (segment (start 146.726 104.399) (end 145.925 105.2) (width 0.2) (layer F.Cu) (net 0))
 (segment (start 146.525 104.6) (end 146.525 104.475) (width 0.2) (layer B.Cu) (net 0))
 (segment (start 146.525 102.975) (end 145.325 102.975) (width 0.2) (layer B.Cu) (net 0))
 (segment (start 144.125 102.975) (end 145.325 102.975) (width 0.2) (layer B.Cu) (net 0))
 (segment (start 144.726 102.814) (end 144.726 103.826) (width 0.2) (layer F.Cu) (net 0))
 (segment (start 144.726 103.826) (end 145.325 104.425) (width 0.2) (layer F.Cu) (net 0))
 (segment (start 146.326 102.814) (end 146.326 103.424) (width 0.2) (layer F.Cu) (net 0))
 (segment (start 145.325 102.975) (end 145.325 104.425) (width 0.2) (layer B.Cu) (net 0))
 (via (at 145.325 104.425) (size 0.6) (drill 0.4) (layers F.Cu B.Cu) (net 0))
 (segment (start 142.225 97.15) (end 142.362 97.15) (width 0.2) (layer B.Cu) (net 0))
 (segment (start 142.362 97.15) (end 144.526 99.314) (width 0.2) (layer B.Cu) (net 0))
 (segment (start 143.625 97.15) (end 143.625 98.413) (width 0.2) (layer B.Cu) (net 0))
 (segment (start 143.625 98.413) (end 144.526 99.314) (width 0.2) (layer B.Cu) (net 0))
 (segment (start 146.7 98.425) (end 145.415 98.425) (width 0.2) (layer B.Cu) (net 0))
 (segment (start 145.415 98.425) (end 144.526 99.314) (width 0.2) (layer B.Cu) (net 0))
 (segment (start 146.7 99.8) (end 145.012 99.8) (width 0.2) (layer B.Cu) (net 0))
 (segment (start 145.012 99.8) (end 144.526 99.314) (width 0.2) (layer B.Cu) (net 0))
 (segment (start 145.325 101.475) (end 145.325 100.113) (width 0.2) (layer B.Cu) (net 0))
 (segment (start 145.325 100.113) (end 144.526 99.314) (width 0.2) (layer B.Cu) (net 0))
 (segment (start 142.35 101.325) (end 142.515 101.325) (width 0.2) (layer B.Cu) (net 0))
 (segment (start 142.515 101.325) (end 144.526 99.314) (width 0.2) (layer B.Cu) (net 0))
 (segment (start 142.35 99.3) (end 144.512 99.3) (width 0.2) (layer B.Cu) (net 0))
 (segment (start 144.512 99.3) (end 144.526 99.314) (width 0.2) (layer B.Cu) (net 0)))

